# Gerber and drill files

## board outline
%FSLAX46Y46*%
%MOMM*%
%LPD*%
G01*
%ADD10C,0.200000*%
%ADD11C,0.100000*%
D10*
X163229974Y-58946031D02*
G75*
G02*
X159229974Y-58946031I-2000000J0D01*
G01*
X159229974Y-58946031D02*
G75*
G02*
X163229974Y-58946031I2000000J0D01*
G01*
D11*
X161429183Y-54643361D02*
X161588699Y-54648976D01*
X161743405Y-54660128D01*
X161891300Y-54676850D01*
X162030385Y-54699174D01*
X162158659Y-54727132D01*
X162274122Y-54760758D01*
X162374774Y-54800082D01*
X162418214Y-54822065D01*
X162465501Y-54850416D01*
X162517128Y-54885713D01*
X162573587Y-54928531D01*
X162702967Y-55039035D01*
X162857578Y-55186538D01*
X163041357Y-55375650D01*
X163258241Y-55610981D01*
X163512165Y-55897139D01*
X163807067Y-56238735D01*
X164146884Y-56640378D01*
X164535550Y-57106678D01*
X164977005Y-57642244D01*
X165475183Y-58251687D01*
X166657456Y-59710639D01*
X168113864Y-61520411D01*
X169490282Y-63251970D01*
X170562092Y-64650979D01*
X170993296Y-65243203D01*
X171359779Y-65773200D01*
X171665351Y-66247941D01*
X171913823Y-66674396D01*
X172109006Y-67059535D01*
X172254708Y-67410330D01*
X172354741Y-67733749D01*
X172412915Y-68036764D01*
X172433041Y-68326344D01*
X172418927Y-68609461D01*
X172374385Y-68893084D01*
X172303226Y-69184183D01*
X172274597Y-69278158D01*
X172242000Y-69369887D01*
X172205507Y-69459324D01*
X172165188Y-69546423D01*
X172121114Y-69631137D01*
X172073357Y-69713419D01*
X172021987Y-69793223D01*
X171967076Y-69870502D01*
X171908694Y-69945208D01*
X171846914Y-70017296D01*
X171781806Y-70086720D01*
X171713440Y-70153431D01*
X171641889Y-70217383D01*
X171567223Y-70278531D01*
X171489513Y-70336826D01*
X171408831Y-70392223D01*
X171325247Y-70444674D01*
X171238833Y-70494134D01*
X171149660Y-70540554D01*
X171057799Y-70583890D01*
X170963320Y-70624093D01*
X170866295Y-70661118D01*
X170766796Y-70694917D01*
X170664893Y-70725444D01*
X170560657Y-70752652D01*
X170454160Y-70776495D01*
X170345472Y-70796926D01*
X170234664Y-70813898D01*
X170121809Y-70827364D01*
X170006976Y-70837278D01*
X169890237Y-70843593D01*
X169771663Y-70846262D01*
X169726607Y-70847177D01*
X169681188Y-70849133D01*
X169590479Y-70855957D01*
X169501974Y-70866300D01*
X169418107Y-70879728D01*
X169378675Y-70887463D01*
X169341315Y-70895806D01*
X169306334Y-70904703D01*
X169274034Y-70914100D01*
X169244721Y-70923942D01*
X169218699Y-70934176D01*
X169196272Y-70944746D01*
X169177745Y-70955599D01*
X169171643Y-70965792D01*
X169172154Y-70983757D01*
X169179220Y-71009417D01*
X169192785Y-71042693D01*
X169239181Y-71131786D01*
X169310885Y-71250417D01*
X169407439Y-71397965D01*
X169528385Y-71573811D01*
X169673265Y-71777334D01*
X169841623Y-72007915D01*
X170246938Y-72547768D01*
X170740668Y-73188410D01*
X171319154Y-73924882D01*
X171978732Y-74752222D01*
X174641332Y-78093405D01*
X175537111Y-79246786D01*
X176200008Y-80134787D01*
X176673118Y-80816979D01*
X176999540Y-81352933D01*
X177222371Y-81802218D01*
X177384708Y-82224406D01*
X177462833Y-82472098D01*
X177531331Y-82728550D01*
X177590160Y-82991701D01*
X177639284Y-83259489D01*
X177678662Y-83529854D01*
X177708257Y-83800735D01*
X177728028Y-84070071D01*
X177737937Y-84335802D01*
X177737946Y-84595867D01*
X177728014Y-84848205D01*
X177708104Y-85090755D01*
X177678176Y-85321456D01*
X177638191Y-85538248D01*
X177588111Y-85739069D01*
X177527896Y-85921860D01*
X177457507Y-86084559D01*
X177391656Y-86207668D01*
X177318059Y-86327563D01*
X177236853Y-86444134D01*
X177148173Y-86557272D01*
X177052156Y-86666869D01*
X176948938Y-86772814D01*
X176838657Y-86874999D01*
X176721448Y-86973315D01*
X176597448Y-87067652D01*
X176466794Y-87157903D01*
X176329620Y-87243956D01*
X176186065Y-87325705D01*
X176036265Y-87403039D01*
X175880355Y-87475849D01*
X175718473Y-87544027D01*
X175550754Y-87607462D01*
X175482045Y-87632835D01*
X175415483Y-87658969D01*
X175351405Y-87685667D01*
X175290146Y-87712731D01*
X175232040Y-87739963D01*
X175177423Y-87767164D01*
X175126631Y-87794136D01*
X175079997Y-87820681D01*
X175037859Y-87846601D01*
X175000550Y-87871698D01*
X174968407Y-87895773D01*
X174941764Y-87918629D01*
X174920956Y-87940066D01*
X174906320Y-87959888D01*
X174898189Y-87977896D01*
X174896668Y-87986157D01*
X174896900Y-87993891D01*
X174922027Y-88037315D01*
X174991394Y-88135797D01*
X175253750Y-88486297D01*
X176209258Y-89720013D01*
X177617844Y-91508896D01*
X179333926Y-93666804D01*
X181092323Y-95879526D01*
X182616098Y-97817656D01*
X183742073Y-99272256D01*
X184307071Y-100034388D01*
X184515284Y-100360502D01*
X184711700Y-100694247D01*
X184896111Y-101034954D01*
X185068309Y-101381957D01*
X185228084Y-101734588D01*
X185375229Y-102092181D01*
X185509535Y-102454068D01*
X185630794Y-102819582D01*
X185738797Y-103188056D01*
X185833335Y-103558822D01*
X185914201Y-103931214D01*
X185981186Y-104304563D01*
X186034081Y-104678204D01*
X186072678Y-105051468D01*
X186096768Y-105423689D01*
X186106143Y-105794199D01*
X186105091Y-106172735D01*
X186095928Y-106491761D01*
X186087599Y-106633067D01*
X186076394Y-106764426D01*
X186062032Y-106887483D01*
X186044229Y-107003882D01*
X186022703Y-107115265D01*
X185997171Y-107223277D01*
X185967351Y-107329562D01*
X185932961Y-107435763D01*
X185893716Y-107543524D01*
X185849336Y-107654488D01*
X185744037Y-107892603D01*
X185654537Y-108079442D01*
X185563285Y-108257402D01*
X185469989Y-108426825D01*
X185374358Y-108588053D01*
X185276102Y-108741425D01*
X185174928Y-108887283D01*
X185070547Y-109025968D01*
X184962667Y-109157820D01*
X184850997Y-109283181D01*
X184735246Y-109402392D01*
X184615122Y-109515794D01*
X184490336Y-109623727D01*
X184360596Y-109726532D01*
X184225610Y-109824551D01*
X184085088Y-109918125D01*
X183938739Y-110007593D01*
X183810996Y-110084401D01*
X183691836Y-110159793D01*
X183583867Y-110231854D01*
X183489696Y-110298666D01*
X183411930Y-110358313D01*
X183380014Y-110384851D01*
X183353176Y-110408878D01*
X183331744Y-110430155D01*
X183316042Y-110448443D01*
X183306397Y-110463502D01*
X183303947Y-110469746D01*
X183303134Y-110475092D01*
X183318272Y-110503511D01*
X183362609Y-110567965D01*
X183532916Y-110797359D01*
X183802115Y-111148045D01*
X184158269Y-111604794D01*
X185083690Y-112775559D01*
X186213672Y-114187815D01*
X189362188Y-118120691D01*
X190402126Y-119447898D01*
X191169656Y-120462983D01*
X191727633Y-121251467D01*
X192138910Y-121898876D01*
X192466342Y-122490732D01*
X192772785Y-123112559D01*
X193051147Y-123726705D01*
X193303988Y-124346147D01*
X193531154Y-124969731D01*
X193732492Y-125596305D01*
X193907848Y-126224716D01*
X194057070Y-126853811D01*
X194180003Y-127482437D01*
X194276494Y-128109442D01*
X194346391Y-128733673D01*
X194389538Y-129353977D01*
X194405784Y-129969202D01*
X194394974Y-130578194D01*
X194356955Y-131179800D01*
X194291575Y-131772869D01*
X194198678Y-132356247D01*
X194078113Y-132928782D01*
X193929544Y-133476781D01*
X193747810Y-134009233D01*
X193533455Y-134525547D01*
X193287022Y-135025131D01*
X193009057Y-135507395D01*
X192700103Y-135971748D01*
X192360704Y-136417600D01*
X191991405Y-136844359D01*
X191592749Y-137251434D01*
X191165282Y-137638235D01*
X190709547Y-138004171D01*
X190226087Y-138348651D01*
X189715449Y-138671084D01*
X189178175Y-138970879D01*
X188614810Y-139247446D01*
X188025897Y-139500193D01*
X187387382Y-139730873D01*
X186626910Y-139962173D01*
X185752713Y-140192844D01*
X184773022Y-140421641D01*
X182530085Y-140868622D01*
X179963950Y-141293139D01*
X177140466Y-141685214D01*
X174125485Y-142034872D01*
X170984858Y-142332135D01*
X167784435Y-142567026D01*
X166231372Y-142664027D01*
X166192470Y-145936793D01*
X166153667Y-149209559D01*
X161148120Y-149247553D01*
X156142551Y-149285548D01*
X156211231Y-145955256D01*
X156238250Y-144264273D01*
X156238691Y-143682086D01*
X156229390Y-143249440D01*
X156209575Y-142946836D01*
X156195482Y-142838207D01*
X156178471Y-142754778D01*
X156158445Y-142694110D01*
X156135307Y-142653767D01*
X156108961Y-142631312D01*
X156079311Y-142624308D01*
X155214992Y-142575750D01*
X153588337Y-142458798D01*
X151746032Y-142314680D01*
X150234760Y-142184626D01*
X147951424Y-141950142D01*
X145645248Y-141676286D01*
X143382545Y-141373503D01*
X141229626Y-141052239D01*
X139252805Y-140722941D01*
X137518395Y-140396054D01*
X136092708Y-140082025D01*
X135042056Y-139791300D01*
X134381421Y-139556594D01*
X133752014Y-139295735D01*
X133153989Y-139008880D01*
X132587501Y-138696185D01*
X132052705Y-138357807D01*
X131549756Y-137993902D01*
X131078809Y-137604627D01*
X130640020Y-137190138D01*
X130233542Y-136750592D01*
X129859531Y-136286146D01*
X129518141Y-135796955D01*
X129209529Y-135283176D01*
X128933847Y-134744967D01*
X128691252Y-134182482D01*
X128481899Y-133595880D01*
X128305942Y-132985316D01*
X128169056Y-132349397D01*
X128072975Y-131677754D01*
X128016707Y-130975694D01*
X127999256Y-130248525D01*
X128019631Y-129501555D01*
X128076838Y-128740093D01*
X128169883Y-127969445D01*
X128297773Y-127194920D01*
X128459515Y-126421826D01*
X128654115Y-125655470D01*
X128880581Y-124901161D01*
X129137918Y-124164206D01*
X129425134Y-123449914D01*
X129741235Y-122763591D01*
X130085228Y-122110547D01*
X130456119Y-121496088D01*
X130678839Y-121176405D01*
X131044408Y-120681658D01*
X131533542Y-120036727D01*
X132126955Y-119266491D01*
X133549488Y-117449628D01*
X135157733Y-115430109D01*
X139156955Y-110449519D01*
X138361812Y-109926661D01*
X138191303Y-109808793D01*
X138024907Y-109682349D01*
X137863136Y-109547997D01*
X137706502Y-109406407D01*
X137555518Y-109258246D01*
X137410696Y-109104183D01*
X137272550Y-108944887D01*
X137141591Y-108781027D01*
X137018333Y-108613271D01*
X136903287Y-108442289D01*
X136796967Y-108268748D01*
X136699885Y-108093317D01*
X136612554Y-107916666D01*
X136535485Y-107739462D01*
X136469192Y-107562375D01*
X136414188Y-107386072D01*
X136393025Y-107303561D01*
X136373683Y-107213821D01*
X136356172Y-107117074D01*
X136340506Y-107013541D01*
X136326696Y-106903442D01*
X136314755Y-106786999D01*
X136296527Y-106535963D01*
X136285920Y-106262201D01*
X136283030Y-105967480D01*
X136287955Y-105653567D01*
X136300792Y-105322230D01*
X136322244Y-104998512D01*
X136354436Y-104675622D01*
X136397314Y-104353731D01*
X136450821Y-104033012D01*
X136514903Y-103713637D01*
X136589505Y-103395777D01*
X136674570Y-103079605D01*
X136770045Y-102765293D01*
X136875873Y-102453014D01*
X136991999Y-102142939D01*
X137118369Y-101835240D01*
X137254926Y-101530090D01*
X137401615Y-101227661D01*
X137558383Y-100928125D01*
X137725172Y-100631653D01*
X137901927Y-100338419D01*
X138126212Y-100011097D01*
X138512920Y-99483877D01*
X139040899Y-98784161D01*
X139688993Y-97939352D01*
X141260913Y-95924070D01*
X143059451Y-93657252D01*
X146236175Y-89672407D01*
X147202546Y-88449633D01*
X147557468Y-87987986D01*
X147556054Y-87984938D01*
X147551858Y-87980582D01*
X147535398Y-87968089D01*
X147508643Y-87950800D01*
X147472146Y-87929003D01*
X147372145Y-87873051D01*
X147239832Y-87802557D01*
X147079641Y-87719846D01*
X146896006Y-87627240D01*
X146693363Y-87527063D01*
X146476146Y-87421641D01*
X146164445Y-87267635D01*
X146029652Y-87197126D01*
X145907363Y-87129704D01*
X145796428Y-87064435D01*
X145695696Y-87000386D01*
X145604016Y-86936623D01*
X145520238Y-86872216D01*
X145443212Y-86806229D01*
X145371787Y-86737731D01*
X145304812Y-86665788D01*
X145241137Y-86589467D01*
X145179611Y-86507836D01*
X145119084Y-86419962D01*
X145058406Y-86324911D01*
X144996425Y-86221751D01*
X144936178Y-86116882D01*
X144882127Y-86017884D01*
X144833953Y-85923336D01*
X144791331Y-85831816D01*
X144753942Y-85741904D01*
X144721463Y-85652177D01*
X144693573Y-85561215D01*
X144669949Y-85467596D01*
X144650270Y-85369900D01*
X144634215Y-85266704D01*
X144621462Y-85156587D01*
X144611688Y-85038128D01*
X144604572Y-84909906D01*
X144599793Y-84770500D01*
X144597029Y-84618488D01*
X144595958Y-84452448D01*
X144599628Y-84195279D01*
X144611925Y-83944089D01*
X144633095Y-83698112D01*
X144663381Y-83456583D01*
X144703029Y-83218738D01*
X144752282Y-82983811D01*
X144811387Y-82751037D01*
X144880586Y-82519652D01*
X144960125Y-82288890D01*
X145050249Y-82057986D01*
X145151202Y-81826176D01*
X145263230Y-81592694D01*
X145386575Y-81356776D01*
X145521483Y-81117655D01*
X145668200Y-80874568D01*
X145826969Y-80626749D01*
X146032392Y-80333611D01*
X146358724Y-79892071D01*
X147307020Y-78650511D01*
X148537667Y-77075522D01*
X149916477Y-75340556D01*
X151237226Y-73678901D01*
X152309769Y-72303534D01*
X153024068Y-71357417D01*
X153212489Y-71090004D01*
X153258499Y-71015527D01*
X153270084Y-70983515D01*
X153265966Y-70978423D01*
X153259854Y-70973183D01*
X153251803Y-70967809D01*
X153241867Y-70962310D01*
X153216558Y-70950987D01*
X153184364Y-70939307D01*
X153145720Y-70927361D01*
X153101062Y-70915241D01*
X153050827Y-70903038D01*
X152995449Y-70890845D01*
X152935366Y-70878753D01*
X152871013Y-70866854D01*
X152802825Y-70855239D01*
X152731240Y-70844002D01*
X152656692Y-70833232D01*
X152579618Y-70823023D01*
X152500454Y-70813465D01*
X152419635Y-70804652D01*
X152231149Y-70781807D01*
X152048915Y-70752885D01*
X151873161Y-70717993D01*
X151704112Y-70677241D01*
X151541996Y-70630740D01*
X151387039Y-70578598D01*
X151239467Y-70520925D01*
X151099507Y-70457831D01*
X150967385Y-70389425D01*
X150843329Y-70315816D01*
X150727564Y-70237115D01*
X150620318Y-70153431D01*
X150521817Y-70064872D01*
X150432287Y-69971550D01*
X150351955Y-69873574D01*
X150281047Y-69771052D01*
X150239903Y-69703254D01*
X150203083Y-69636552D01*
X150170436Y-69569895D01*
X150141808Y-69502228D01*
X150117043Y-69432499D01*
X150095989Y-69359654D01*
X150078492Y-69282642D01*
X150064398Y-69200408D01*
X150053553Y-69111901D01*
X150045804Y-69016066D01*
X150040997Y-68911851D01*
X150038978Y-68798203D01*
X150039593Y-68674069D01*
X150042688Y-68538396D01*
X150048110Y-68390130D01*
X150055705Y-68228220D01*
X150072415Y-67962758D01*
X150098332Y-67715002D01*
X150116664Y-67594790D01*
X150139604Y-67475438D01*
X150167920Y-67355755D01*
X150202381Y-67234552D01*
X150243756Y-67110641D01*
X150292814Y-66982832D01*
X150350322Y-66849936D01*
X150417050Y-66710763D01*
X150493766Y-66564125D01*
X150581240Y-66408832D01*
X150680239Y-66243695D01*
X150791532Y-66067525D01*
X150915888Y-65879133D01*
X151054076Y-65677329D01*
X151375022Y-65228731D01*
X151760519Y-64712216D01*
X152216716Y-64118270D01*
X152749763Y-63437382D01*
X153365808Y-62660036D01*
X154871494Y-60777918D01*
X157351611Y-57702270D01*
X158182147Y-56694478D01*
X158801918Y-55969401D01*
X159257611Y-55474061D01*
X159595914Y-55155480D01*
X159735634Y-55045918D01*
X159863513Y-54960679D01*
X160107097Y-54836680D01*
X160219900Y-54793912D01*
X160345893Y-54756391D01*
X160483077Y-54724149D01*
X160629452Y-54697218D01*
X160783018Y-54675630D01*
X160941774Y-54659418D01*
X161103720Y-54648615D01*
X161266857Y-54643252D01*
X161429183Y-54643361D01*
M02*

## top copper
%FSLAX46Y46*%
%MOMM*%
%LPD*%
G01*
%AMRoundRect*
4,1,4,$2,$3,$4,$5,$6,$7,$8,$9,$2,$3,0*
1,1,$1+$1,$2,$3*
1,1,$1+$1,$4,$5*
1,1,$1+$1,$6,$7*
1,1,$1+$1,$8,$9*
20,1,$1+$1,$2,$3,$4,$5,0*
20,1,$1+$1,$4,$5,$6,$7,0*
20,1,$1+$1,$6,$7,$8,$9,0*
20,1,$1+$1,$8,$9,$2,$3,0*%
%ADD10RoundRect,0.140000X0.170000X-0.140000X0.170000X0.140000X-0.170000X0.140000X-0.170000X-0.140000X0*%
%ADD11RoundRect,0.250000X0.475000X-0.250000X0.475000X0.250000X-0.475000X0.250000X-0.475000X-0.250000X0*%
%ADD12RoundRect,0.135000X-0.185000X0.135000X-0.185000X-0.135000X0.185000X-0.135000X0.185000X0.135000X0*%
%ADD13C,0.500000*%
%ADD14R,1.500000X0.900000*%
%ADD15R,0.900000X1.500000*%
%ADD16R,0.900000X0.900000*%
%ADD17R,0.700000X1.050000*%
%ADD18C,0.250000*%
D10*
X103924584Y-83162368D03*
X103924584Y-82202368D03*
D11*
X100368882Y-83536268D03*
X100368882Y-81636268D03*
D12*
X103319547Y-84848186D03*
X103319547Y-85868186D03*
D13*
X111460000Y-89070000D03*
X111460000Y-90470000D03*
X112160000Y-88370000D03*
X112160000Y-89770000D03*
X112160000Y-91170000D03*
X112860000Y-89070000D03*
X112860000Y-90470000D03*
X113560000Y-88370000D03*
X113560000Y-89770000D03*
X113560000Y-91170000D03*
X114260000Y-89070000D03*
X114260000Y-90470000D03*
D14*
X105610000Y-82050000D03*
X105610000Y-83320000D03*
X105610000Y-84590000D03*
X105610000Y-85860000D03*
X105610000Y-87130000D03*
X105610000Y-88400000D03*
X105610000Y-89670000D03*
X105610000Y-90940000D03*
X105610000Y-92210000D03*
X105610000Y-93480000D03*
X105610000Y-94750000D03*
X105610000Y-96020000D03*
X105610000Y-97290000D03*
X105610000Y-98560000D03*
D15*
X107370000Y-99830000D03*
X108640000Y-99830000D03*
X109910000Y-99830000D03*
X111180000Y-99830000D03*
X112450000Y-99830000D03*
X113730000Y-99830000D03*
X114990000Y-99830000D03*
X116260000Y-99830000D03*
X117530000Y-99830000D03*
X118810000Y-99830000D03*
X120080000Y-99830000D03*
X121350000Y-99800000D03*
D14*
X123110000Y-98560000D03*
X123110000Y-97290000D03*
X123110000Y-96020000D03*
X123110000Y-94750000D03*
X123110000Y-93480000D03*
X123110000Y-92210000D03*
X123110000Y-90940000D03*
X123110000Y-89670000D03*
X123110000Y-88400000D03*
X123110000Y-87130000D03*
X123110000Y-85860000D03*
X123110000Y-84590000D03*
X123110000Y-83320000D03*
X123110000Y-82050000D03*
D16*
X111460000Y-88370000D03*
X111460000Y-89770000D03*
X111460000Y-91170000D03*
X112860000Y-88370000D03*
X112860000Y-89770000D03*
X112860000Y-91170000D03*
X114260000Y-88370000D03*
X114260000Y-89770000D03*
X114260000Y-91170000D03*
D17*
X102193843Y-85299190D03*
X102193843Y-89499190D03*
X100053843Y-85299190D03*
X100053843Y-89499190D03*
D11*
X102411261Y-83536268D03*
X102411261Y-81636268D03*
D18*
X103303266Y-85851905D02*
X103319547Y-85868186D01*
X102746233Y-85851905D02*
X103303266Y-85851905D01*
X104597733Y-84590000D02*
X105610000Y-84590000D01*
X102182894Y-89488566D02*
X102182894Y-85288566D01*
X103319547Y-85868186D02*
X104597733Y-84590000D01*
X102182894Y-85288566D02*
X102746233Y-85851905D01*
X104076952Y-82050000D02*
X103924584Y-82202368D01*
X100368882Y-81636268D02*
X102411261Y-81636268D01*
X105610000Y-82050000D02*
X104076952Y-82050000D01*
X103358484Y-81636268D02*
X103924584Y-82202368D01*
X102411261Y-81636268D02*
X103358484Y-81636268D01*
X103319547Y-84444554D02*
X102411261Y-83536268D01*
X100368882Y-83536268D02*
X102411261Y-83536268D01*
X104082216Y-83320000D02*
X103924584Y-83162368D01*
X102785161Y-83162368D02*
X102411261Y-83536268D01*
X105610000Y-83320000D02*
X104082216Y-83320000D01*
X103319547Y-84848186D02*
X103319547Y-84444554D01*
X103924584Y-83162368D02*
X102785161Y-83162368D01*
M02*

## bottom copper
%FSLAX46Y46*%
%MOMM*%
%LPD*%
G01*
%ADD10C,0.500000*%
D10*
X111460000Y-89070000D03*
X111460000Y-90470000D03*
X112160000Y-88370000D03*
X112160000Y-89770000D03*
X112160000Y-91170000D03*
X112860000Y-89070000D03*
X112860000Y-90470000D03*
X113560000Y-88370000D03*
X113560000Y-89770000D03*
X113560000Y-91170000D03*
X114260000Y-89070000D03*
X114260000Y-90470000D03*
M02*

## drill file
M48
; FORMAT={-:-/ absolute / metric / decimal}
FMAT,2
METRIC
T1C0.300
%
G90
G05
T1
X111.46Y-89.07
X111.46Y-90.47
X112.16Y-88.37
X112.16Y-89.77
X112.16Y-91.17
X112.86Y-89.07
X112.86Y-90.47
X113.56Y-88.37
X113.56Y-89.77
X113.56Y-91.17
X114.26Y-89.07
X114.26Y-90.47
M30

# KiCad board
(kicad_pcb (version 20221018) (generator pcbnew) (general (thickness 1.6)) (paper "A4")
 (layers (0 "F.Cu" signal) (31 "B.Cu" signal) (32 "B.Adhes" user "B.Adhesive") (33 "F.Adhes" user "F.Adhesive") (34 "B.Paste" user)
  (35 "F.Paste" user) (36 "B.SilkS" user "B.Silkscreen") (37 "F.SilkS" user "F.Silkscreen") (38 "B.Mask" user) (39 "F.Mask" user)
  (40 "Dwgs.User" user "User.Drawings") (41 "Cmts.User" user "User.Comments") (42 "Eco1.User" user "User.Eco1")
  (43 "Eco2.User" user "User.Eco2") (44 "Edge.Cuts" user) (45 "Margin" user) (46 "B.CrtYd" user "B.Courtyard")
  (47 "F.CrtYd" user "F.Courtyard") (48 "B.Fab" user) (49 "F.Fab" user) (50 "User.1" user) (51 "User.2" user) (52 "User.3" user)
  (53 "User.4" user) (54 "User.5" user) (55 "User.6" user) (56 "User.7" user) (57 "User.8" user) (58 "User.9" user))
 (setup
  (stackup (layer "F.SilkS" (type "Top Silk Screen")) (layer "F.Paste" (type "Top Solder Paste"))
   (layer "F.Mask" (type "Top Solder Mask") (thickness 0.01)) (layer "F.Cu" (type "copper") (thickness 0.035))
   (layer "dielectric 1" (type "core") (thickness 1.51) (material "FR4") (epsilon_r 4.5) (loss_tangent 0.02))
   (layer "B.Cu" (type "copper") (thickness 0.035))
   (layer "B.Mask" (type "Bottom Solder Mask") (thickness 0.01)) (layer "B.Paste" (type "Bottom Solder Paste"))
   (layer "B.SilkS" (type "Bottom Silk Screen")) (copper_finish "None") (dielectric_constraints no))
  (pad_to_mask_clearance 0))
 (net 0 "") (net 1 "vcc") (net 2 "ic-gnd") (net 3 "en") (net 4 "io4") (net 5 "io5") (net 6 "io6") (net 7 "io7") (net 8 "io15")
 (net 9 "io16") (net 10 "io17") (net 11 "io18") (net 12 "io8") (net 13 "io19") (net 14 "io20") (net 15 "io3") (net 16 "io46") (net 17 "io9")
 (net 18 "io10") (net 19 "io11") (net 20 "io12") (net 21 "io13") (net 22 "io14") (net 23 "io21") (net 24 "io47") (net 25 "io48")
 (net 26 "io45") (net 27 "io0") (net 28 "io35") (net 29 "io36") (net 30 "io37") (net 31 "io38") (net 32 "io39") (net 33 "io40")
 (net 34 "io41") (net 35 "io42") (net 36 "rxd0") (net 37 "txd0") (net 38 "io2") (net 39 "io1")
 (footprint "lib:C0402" (layer "F.Cu") (at 103.924584 82.682368 90)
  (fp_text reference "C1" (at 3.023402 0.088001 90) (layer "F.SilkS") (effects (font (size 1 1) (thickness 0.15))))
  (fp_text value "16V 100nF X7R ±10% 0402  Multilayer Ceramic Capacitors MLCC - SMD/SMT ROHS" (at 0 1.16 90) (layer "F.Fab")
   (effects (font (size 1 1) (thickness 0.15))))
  (pad "1" smd roundrect (at -0.48 0 90) (size 0.56 0.62) (layers "F.Cu" "F.Paste" "F.Mask") (roundrect_rratio 0.25) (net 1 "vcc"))
  (pad "2" smd roundrect (at 0.48 0 90) (size 0.56 0.62) (layers "F.Cu" "F.Paste" "F.Mask") (roundrect_rratio 0.25) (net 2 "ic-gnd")))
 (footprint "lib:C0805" (layer "F.Cu") (at 100.368882 82.586268 90)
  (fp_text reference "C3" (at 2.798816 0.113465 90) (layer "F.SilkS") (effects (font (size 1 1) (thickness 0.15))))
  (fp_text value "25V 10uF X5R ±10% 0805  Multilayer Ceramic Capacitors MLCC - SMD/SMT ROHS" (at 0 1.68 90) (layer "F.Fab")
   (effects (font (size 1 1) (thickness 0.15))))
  (pad "1" smd roundrect (at -0.95 0 90) (size 1 1.45) (layers "F.Cu" "F.Paste" "F.Mask") (roundrect_rratio 0.25) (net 1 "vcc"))
  (pad "2" smd roundrect (at 0.95 0 90) (size 1 1.45) (layers "F.Cu" "F.Paste" "F.Mask") (roundrect_rratio 0.25) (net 2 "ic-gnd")))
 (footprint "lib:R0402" (layer "F.Cu") (at 103.319547 85.358186 -90)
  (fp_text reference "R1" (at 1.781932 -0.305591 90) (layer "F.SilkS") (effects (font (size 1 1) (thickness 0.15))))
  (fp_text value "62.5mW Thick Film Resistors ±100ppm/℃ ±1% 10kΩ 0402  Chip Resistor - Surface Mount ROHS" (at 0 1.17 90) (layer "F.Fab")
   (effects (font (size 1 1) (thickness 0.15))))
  (pad "1" smd roundrect (at -0.51 0 270) (size 0.54 0.64) (layers "F.Cu" "F.Paste" "F.Mask") (roundrect_rratio 0.25) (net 1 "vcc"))
  (pad "2" smd roundrect (at 0.51 0 270) (size 0.54 0.64) (layers "F.Cu" "F.Paste" "F.Mask") (roundrect_rratio 0.25) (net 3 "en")))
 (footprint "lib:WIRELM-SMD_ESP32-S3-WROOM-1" (layer "F.Cu") (at 114.36 90.94)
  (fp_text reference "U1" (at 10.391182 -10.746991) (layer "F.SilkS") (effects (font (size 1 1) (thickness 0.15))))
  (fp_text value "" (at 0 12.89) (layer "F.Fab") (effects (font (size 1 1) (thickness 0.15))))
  (pad "" thru_hole circle (at -2.9 -1.87) (size 0.5 0.5) (drill 0.3) (layers "*.Cu" "*.Paste" "*.Mask"))
  (pad "" thru_hole circle (at -2.9 -0.47) (size 0.5 0.5) (drill 0.3) (layers "*.Cu" "*.Paste" "*.Mask"))
  (pad "" thru_hole circle (at -2.2 -2.57) (size 0.5 0.5) (drill 0.3) (layers "*.Cu" "*.Paste" "*.Mask"))
  (pad "" thru_hole circle (at -2.2 -1.17) (size 0.5 0.5) (drill 0.3) (layers "*.Cu" "*.Paste" "*.Mask"))
  (pad "" thru_hole circle (at -2.2 0.23) (size 0.5 0.5) (drill 0.3) (layers "*.Cu" "*.Paste" "*.Mask"))
  (pad "" thru_hole circle (at -1.5 -1.87) (size 0.5 0.5) (drill 0.3) (layers "*.Cu" "*.Paste" "*.Mask"))
  (pad "" thru_hole circle (at -1.5 -0.47) (size 0.5 0.5) (drill 0.3) (layers "*.Cu" "*.Paste" "*.Mask"))
  (pad "" thru_hole circle (at -0.8 -2.57) (size 0.5 0.5) (drill 0.3) (layers "*.Cu" "*.Paste" "*.Mask"))
  (pad "" thru_hole circle (at -0.8 -1.17) (size 0.5 0.5) (drill 0.3) (layers "*.Cu" "*.Paste" "*.Mask"))
  (pad "" thru_hole circle (at -0.8 0.23) (size 0.5 0.5) (drill 0.3) (layers "*.Cu" "*.Paste" "*.Mask"))
  (pad "" thru_hole circle (at -0.1 -1.87) (size 0.5 0.5) (drill 0.3) (layers "*.Cu" "*.Paste" "*.Mask"))
  (pad "" thru_hole circle (at -0.1 -0.47) (size 0.5 0.5) (drill 0.3) (layers "*.Cu" "*.Paste" "*.Mask"))
  (pad "1" smd rect (at -8.75 -8.89) (size 1.5 0.9) (layers "F.Cu" "F.Paste" "F.Mask") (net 2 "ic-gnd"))
  (pad "2" smd rect (at -8.75 -7.62) (size 1.5 0.9) (layers "F.Cu" "F.Paste" "F.Mask") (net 1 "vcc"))
  (pad "3" smd rect (at -8.75 -6.35) (size 1.5 0.9) (layers "F.Cu" "F.Paste" "F.Mask") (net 3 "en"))
  (pad "4" smd rect (at -8.75 -5.08) (size 1.5 0.9) (layers "F.Cu" "F.Paste" "F.Mask") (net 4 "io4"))
  (pad "5" smd rect (at -8.75 -3.81) (size 1.5 0.9) (layers "F.Cu" "F.Paste" "F.Mask") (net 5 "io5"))
  (pad "6" smd rect (at -8.75 -2.54) (size 1.5 0.9) (layers "F.Cu" "F.Paste" "F.Mask") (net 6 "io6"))
  (pad "7" smd rect (at -8.75 -1.27) (size 1.5 0.9) (layers "F.Cu" "F.Paste" "F.Mask") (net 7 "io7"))
  (pad "8" smd rect (at -8.75 0) (size 1.5 0.9) (layers "F.Cu" "F.Paste" "F.Mask") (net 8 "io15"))
  (pad "9" smd rect (at -8.75 1.27) (size 1.5 0.9) (layers "F.Cu" "F.Paste" "F.Mask") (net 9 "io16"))
  (pad "10" smd rect (at -8.75 2.54) (size 1.5 0.9) (layers "F.Cu" "F.Paste" "F.Mask") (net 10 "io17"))
  (pad "11" smd rect (at -8.75 3.81) (size 1.5 0.9) (layers "F.Cu" "F.Paste" "F.Mask") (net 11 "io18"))
  (pad "12" smd rect (at -8.75 5.08) (size 1.5 0.9) (layers "F.Cu" "F.Paste" "F.Mask") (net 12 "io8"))
  (pad "13" smd rect (at -8.75 6.35) (size 1.5 0.9) (layers "F.Cu" "F.Paste" "F.Mask") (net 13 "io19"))
  (pad "14" smd rect (at -8.75 7.62) (size 1.5 0.9) (layers "F.Cu" "F.Paste" "F.Mask") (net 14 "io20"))
  (pad "15" smd rect (at -6.99 8.89 90) (size 1.5 0.9) (layers "F.Cu" "F.Paste" "F.Mask") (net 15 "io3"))
  (pad "16" smd rect (at -5.72 8.89 90) (size 1.5 0.9) (layers "F.Cu" "F.Paste" "F.Mask") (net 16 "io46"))
  (pad "17" smd rect (at -4.45 8.89 90) (size 1.5 0.9) (layers "F.Cu" "F.Paste" "F.Mask") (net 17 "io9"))
  (pad "18" smd rect (at -3.18 8.89 90) (size 1.5 0.9) (layers "F.Cu" "F.Paste" "F.Mask") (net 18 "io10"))
  (pad "19" smd rect (at -1.91 8.89 90) (size 1.5 0.9) (layers "F.Cu" "F.Paste" "F.Mask") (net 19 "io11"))
  (pad "20" smd rect (at -0.63 8.89 90) (size 1.5 0.9) (layers "F.Cu" "F.Paste" "F.Mask") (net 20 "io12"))
  (pad "21" smd rect (at 0.63 8.89 90) (size 1.5 0.9) (layers "F.Cu" "F.Paste" "F.Mask") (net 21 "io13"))
  (pad "22" smd rect (at 1.9 8.89 90) (size 1.5 0.9) (layers "F.Cu" "F.Paste" "F.Mask") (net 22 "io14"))
  (pad "23" smd rect (at 3.17 8.89 90) (size 1.5 0.9) (layers "F.Cu" "F.Paste" "F.Mask") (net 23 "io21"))
  (pad "24" smd rect (at 4.45 8.89 90) (size 1.5 0.9) (layers "F.Cu" "F.Paste" "F.Mask") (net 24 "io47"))
  (pad "25" smd rect (at 5.72 8.89 90) (size 1.5 0.9) (layers "F.Cu" "F.Paste" "F.Mask") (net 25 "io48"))
  (pad "26" smd rect (at 6.99 8.86 90) (size 1.5 0.9) (layers "F.Cu" "F.Paste" "F.Mask") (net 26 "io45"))
  (pad "27" smd rect (at 8.75 7.62 180) (size 1.5 0.9) (layers "F.Cu" "F.Paste" "F.Mask") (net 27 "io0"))
  (pad "28" smd rect (at 8.75 6.35 180) (size 1.5 0.9) (layers "F.Cu" "F.Paste" "F.Mask") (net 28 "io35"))
  (pad "29" smd rect (at 8.75 5.08 180) (size 1.5 0.9) (layers "F.Cu" "F.Paste" "F.Mask") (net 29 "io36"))
  (pad "30" smd rect (at 8.75 3.81 180) (size 1.5 0.9) (layers "F.Cu" "F.Paste" "F.Mask") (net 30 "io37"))
  (pad "31" smd rect (at 8.75 2.54 180) (size 1.5 0.9) (layers "F.Cu" "F.Paste" "F.Mask") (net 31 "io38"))
  (pad "32" smd rect (at 8.75 1.27 180) (size 1.5 0.9) (layers "F.Cu" "F.Paste" "F.Mask") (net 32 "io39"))
  (pad "33" smd rect (at 8.75 0 180) (size 1.5 0.9) (layers "F.Cu" "F.Paste" "F.Mask") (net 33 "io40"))
  (pad "34" smd rect (at 8.75 -1.27 180) (size 1.5 0.9) (layers "F.Cu" "F.Paste" "F.Mask") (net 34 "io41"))
  (pad "35" smd rect (at 8.75 -2.54 180) (size 1.5 0.9) (layers "F.Cu" "F.Paste" "F.Mask") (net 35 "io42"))
  (pad "36" smd rect (at 8.75 -3.81 180) (size 1.5 0.9) (layers "F.Cu" "F.Paste" "F.Mask") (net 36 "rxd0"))
  (pad "37" smd rect (at 8.75 -5.08 180) (size 1.5 0.9) (layers "F.Cu" "F.Paste" "F.Mask") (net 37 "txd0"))
  (pad "38" smd rect (at 8.75 -6.35 180) (size 1.5 0.9) (layers "F.Cu" "F.Paste" "F.Mask") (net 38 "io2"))
  (pad "39" smd rect (at 8.75 -7.62 180) (size 1.5 0.9) (layers "F.Cu" "F.Paste" "F.Mask") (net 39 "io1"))
  (pad "40" smd rect (at 8.75 -8.89 180) (size 1.5 0.9) (layers "F.Cu" "F.Paste" "F.Mask") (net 2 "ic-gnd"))
  (pad "41" smd rect (at -2.9 -2.57 90) (size 0.9 0.9) (layers "F.Cu" "F.Paste" "F.Mask") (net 2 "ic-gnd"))
  (pad "41" smd rect (at -2.9 -1.17 90) (size 0.9 0.9) (layers "F.Cu" "F.Paste" "F.Mask") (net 2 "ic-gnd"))
  (pad "41" smd rect (at -2.9 0.23 90) (size 0.9 0.9) (layers "F.Cu" "F.Paste" "F.Mask") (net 2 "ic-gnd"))
  (pad "41" smd rect (at -1.5 -2.57 90) (size 0.9 0.9) (layers "F.Cu" "F.Paste" "F.Mask") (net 2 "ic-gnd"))
  (pad "41" smd rect (at -1.5 -1.17 90) (size 0.9 0.9) (layers "F.Cu" "F.Paste" "F.Mask") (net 2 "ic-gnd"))
  (pad "41" smd rect (at -1.5 0.23 90) (size 0.9 0.9) (layers "F.Cu" "F.Paste" "F.Mask") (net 2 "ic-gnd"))
  (pad "41" smd rect (at -0.1 -2.57 90) (size 0.9 0.9) (layers "F.Cu" "F.Paste" "F.Mask") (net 2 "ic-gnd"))
  (pad "41" smd rect (at -0.1 -1.17 90) (size 0.9 0.9) (layers "F.Cu" "F.Paste" "F.Mask") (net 2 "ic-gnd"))
  (pad "41" smd rect (at -0.1 0.23 90) (size 0.9 0.9) (layers "F.Cu" "F.Paste" "F.Mask") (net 2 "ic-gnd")))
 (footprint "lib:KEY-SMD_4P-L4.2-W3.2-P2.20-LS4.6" (layer "F.Cu") (at 101.123843 87.39919 -90)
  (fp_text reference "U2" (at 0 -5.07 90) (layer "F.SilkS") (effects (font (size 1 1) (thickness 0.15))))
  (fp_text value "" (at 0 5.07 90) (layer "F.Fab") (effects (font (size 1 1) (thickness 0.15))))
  (pad "1" smd rect (at -2.1 -1.07 270) (size 1.05 0.7) (layers "F.Cu" "F.Paste" "F.Mask") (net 3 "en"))
  (pad "2" smd rect (at 2.1 -1.07 270) (size 1.05 0.7) (layers "F.Cu" "F.Paste" "F.Mask") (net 3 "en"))
  (pad "3" smd rect (at -2.1 1.07 270) (size 1.05 0.7) (layers "F.Cu" "F.Paste" "F.Mask") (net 2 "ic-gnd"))
  (pad "4" smd rect (at 2.1 1.07 270) (size 1.05 0.7) (layers "F.Cu" "F.Paste" "F.Mask") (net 2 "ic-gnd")))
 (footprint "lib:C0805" (layer "F.Cu") (at 102.411261 82.586268 90)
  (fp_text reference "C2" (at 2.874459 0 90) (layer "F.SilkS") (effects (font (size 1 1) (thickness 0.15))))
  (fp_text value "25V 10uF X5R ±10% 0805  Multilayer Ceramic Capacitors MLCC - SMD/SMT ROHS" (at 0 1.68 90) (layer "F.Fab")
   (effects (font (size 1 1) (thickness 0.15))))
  (pad "1" smd roundrect (at -0.95 0 90) (size 1 1.45) (layers "F.Cu" "F.Paste" "F.Mask") (roundrect_rratio 0.25) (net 1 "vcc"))
  (pad "2" smd roundrect (at 0.95 0 90) (size 1 1.45) (layers "F.Cu" "F.Paste" "F.Mask") (roundrect_rratio 0.25) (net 2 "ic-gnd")))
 (gr_circle (center 161.229974 58.946031) (end 163.229974 58.946031) (stroke (width 0.2) (type default)) (fill none) (layer "Edge.Cuts"))
 (gr_poly
  (pts (xy 161.429183 54.643361) (xy 161.588699 54.648976) (xy 161.743405 54.660128) (xy 161.8913 54.67685) (xy 162.030385 54.699174)
   (xy 162.158659 54.727132) (xy 162.274122 54.760758) (xy 162.374774 54.800082) (xy 162.418214 54.822065) (xy 162.465501 54.850416)
   (xy 162.517128 54.885713) (xy 162.573587 54.928531) (xy 162.702967 55.039035) (xy 162.857578 55.186538) (xy 163.041357 55.37565)
   (xy 163.258241 55.610981) (xy 163.512165 55.897139) (xy 163.807067 56.238735) (xy 164.146884 56.640378) (xy 164.53555 57.106678)
   (xy 164.977005 57.642244) (xy 165.475183 58.251687) (xy 166.657456 59.710639) (xy 168.113864 61.520411) (xy 169.490282 63.25197)
   (xy 170.562092 64.650979) (xy 170.993296 65.243203) (xy 171.359779 65.7732) (xy 171.665351 66.247941) (xy 171.913823 66.674396)
   (xy 172.109006 67.059535) (xy 172.254708 67.41033) (xy 172.354741 67.733749) (xy 172.412915 68.036764) (xy 172.433041 68.326344)
   (xy 172.418927 68.609461) (xy 172.374385 68.893084) (xy 172.303226 69.184183) (xy 172.274597 69.278158) (xy 172.242 69.369887)
   (xy 172.205507 69.459324) (xy 172.165188 69.546423) (xy 172.121114 69.631137) (xy 172.073357 69.713419) (xy 172.021987 69.793223)
   (xy 171.967076 69.870502) (xy 171.908694 69.945208) (xy 171.846914 70.017296) (xy 171.781806 70.08672) (xy 171.71344 70.153431)
   (xy 171.641889 70.217383) (xy 171.567223 70.278531) (xy 171.489513 70.336826) (xy 171.408831 70.392223) (xy 171.325247 70.444674)
   (xy 171.238833 70.494134) (xy 171.14966 70.540554) (xy 171.057799 70.58389) (xy 170.96332 70.624093) (xy 170.866295 70.661118)
   (xy 170.766796 70.694917) (xy 170.664893 70.725444) (xy 170.560657 70.752652) (xy 170.45416 70.776495) (xy 170.345472 70.796926)
   (xy 170.234664 70.813898) (xy 170.121809 70.827364) (xy 170.006976 70.837278) (xy 169.890237 70.843593) (xy 169.771663 70.846262)
   (xy 169.726607 70.847177) (xy 169.681188 70.849133) (xy 169.590479 70.855957) (xy 169.501974 70.8663) (xy 169.418107 70.879728)
   (xy 169.378675 70.887463) (xy 169.341315 70.895806) (xy 169.306334 70.904703) (xy 169.274034 70.9141) (xy 169.244721 70.923942)
   (xy 169.218699 70.934176) (xy 169.196272 70.944746) (xy 169.177745 70.955599) (xy 169.171643 70.965792) (xy 169.172154 70.983757)
   (xy 169.17922 71.009417) (xy 169.192785 71.042693) (xy 169.239181 71.131786) (xy 169.310885 71.250417) (xy 169.407439 71.397965)
   (xy 169.528385 71.573811) (xy 169.673265 71.777334) (xy 169.841623 72.007915) (xy 170.246938 72.547768) (xy 170.740668 73.18841)
   (xy 171.319154 73.924882) (xy 171.978732 74.752222) (xy 174.641332 78.093405) (xy 175.537111 79.246786) (xy 176.200008 80.134787)
   (xy 176.673118 80.816979) (xy 176.99954 81.352933) (xy 177.222371 81.802218) (xy 177.384708 82.224406) (xy 177.462833 82.472098)
   (xy 177.531331 82.72855) (xy 177.59016 82.991701) (xy 177.639284 83.259489) (xy 177.678662 83.529854) (xy 177.708257 83.800735)
   (xy 177.728028 84.070071) (xy 177.737937 84.335802) (xy 177.737946 84.595867) (xy 177.728014 84.848205) (xy 177.708104 85.090755)
   (xy 177.678176 85.321456) (xy 177.638191 85.538248) (xy 177.588111 85.739069) (xy 177.527896 85.92186) (xy 177.457507 86.084559)
   (xy 177.391656 86.207668) (xy 177.318059 86.327563) (xy 177.236853 86.444134) (xy 177.148173 86.557272) (xy 177.052156 86.666869)
   (xy 176.948938 86.772814) (xy 176.838657 86.874999) (xy 176.721448 86.973315) (xy 176.597448 87.067652) (xy 176.466794 87.157903)
   (xy 176.32962 87.243956) (xy 176.186065 87.325705) (xy 176.036265 87.403039) (xy 175.880355 87.475849) (xy 175.718473 87.544027)
   (xy 175.550754 87.607462) (xy 175.482045 87.632835) (xy 175.415483 87.658969) (xy 175.351405 87.685667) (xy 175.290146 87.712731)
   (xy 175.23204 87.739963) (xy 175.177423 87.767164) (xy 175.126631 87.794136) (xy 175.079997 87.820681) (xy 175.037859 87.846601)
   (xy 175.00055 87.871698) (xy 174.968407 87.895773) (xy 174.941764 87.918629) (xy 174.920956 87.940066) (xy 174.90632 87.959888)
   (xy 174.898189 87.977896) (xy 174.896668 87.986157) (xy 174.8969 87.993891) (xy 174.922027 88.037315) (xy 174.991394 88.135797)
   (xy 175.25375 88.486297) (xy 176.209258 89.720013) (xy 177.617844 91.508896) (xy 179.333926 93.666804) (xy 181.092323 95.879526)
   (xy 182.616098 97.817656) (xy 183.742073 99.272256) (xy 184.307071 100.034388) (xy 184.515284 100.360502) (xy 184.7117 100.694247)
   (xy 184.896111 101.034954) (xy 185.068309 101.381957) (xy 185.228084 101.734588) (xy 185.375229 102.092181) (xy 185.509535 102.454068)
   (xy 185.630794 102.819582) (xy 185.738797 103.188056) (xy 185.833335 103.558822) (xy 185.914201 103.931214) (xy 185.981186 104.304563)
   (xy 186.034081 104.678204) (xy 186.072678 105.051468) (xy 186.096768 105.423689) (xy 186.106143 105.794199) (xy 186.105091 106.172735)
   (xy 186.095928 106.491761) (xy 186.087599 106.633067) (xy 186.076394 106.764426) (xy 186.062032 106.887483) (xy 186.044229 107.003882)
   (xy 186.022703 107.115265) (xy 185.997171 107.223277) (xy 185.967351 107.329562) (xy 185.932961 107.435763) (xy 185.893716 107.543524)
   (xy 185.849336 107.654488) (xy 185.744037 107.892603) (xy 185.654537 108.079442) (xy 185.563285 108.257402) (xy 185.469989 108.426825)
   (xy 185.374358 108.588053) (xy 185.276102 108.741425) (xy 185.174928 108.887283) (xy 185.070547 109.025968) (xy 184.962667 109.15782)
   (xy 184.850997 109.283181) (xy 184.735246 109.402392) (xy 184.615122 109.515794) (xy 184.490336 109.623727) (xy 184.360596 109.726532)
   (xy 184.22561 109.824551) (xy 184.085088 109.918125) (xy 183.938739 110.007593) (xy 183.810996 110.084401) (xy 183.691836 110.159793)
   (xy 183.583867 110.231854) (xy 183.489696 110.298666) (xy 183.41193 110.358313) (xy 183.380014 110.384851) (xy 183.353176 110.408878)
   (xy 183.331744 110.430155) (xy 183.316042 110.448443) (xy 183.306397 110.463502) (xy 183.303947 110.469746) (xy 183.303134 110.475092)
   (xy 183.318272 110.503511) (xy 183.362609 110.567965) (xy 183.532916 110.797359) (xy 183.802115 111.148045) (xy 184.158269 111.604794)
   (xy 185.08369 112.775559) (xy 186.213672 114.187815) (xy 189.362188 118.120691) (xy 190.402126 119.447898) (xy 191.169656 120.462983)
   (xy 191.727633 121.251467) (xy 192.13891 121.898876) (xy 192.466342 122.490732) (xy 192.772785 123.112559) (xy 193.051147 123.726705)
   (xy 193.303988 124.346147) (xy 193.531154 124.969731) (xy 193.732492 125.596305) (xy 193.907848 126.224716) (xy 194.05707 126.853811)
   (xy 194.180003 127.482437) (xy 194.276494 128.109442) (xy 194.346391 128.733673) (xy 194.389538 129.353977) (xy 194.405784 129.969202)
   (xy 194.394974 130.578194) (xy 194.356955 131.1798) (xy 194.291575 131.772869) (xy 194.198678 132.356247) (xy 194.078113 132.928782)
   (xy 193.929544 133.476781) (xy 193.74781 134.009233) (xy 193.533455 134.525547) (xy 193.287022 135.025131) (xy 193.009057 135.507395)
   (xy 192.700103 135.971748) (xy 192.360704 136.4176) (xy 191.991405 136.844359) (xy 191.592749 137.251434) (xy 191.165282 137.638235)
   (xy 190.709547 138.004171) (xy 190.226087 138.348651) (xy 189.715449 138.671084) (xy 189.178175 138.970879) (xy 188.61481 139.247446)
   (xy 188.025897 139.500193) (xy 187.387382 139.730873) (xy 186.62691 139.962173) (xy 185.752713 140.192844) (xy 184.773022 140.421641)
   (xy 182.530085 140.868622) (xy 179.96395 141.293139) (xy 177.140466 141.685214) (xy 174.125485 142.034872) (xy 170.984858 142.332135)
   (xy 167.784435 142.567026) (xy 166.231372 142.664027) (xy 166.19247 145.936793) (xy 166.153667 149.209559) (xy 161.14812 149.247553)
   (xy 156.142551 149.285548) (xy 156.211231 145.955256) (xy 156.23825 144.264273) (xy 156.238691 143.682086) (xy 156.22939 143.24944)
   (xy 156.209575 142.946836) (xy 156.195482 142.838207) (xy 156.178471 142.754778) (xy 156.158445 142.69411) (xy 156.135307 142.653767)
   (xy 156.108961 142.631312) (xy 156.079311 142.624308) (xy 155.214992 142.57575) (xy 153.588337 142.458798) (xy 151.746032 142.31468)
   (xy 150.23476 142.184626) (xy 147.951424 141.950142) (xy 145.645248 141.676286) (xy 143.382545 141.373503) (xy 141.229626 141.052239)
   (xy 139.252805 140.722941) (xy 137.518395 140.396054) (xy 136.092708 140.082025) (xy 135.042056 139.7913) (xy 134.381421 139.556594)
   (xy 133.752014 139.295735) (xy 133.153989 139.00888) (xy 132.587501 138.696185) (xy 132.052705 138.357807) (xy 131.549756 137.993902)
   (xy 131.078809 137.604627) (xy 130.64002 137.190138) (xy 130.233542 136.750592) (xy 129.859531 136.286146) (xy 129.518141 135.796955)
   (xy 129.209529 135.283176) (xy 128.933847 134.744967) (xy 128.691252 134.182482) (xy 128.481899 133.59588) (xy 128.305942 132.985316)
   (xy 128.169056 132.349397) (xy 128.072975 131.677754) (xy 128.016707 130.975694) (xy 127.999256 130.248525) (xy 128.019631 129.501555)
   (xy 128.076838 128.740093) (xy 128.169883 127.969445) (xy 128.297773 127.19492) (xy 128.459515 126.421826) (xy 128.654115 125.65547)
   (xy 128.880581 124.901161) (xy 129.137918 124.164206) (xy 129.425134 123.449914) (xy 129.741235 122.763591) (xy 130.085228 122.110547)
   (xy 130.456119 121.496088) (xy 130.678839 121.176405) (xy 131.044408 120.681658) (xy 131.533542 120.036727) (xy 132.126955 119.266491)
   (xy 133.549488 117.449628) (xy 135.157733 115.430109) (xy 139.156955 110.449519) (xy 138.361812 109.926661) (xy 138.191303 109.808793)
   (xy 138.024907 109.682349) (xy 137.863136 109.547997) (xy 137.706502 109.406407) (xy 137.555518 109.258246) (xy 137.410696 109.104183)
   (xy 137.27255 108.944887) (xy 137.141591 108.781027) (xy 137.018333 108.613271) (xy 136.903287 108.442289) (xy 136.796967 108.268748)
   (xy 136.699885 108.093317) (xy 136.612554 107.916666) (xy 136.535485 107.739462) (xy 136.469192 107.562375) (xy 136.414188 107.386072)
   (xy 136.393025 107.303561) (xy 136.373683 107.213821) (xy 136.356172 107.117074) (xy 136.340506 107.013541) (xy 136.326696 106.903442)
   (xy 136.314755 106.786999) (xy 136.296527 106.535963) (xy 136.28592 106.262201) (xy 136.28303 105.96748) (xy 136.287955 105.653567)
   (xy 136.300792 105.32223) (xy 136.322244 104.998512) (xy 136.354436 104.675622) (xy 136.397314 104.353731) (xy 136.450821 104.033012)
   (xy 136.514903 103.713637) (xy 136.589505 103.395777) (xy 136.67457 103.079605) (xy 136.770045 102.765293) (xy 136.875873 102.453014)
   (xy 136.991999 102.142939) (xy 137.118369 101.83524) (xy 137.254926 101.53009) (xy 137.401615 101.227661) (xy 137.558383 100.928125)
   (xy 137.725172 100.631653) (xy 137.901927 100.338419) (xy 138.126212 100.011097) (xy 138.51292 99.483877) (xy 139.040899 98.784161)
   (xy 139.688993 97.939352) (xy 141.260913 95.92407) (xy 143.059451 93.657252) (xy 146.236175 89.672407) (xy 147.202546 88.449633)
   (xy 147.557468 87.987986) (xy 147.556054 87.984938) (xy 147.551858 87.980582) (xy 147.535398 87.968089) (xy 147.508643 87.9508)
   (xy 147.472146 87.929003) (xy 147.372145 87.873051) (xy 147.239832 87.802557) (xy 147.079641 87.719846) (xy 146.896006 87.62724)
   (xy 146.693363 87.527063) (xy 146.476146 87.421641) (xy 146.164445 87.267635) (xy 146.029652 87.197126) (xy 145.907363 87.129704)
   (xy 145.796428 87.064435) (xy 145.695696 87.000386) (xy 145.604016 86.936623) (xy 145.520238 86.872216) (xy 145.443212 86.806229)
   (xy 145.371787 86.737731) (xy 145.304812 86.665788) (xy 145.241137 86.589467) (xy 145.179611 86.507836) (xy 145.119084 86.419962)
   (xy 145.058406 86.324911) (xy 144.996425 86.221751) (xy 144.936178 86.116882) (xy 144.882127 86.017884) (xy 144.833953 85.923336)
   (xy 144.791331 85.831816) (xy 144.753942 85.741904) (xy 144.721463 85.652177) (xy 144.693573 85.561215) (xy 144.669949 85.467596)
   (xy 144.65027 85.3699) (xy 144.634215 85.266704) (xy 144.621462 85.156587) (xy 144.611688 85.038128) (xy 144.604572 84.909906)
   (xy 144.599793 84.7705) (xy 144.597029 84.618488) (xy 144.595958 84.452448) (xy 144.599628 84.195279) (xy 144.611925 83.944089)
   (xy 144.633095 83.698112) (xy 144.663381 83.456583) (xy 144.703029 83.218738) (xy 144.752282 82.983811) (xy 144.811387 82.751037)
   (xy 144.880586 82.519652) (xy 144.960125 82.28889) (xy 145.050249 82.057986) (xy 145.151202 81.826176) (xy 145.26323 81.592694)
   (xy 145.386575 81.356776) (xy 145.521483 81.117655) (xy 145.6682 80.874568) (xy 145.826969 80.626749) (xy 146.032392 80.333611)
   (xy 146.358724 79.892071) (xy 147.30702 78.650511) (xy 148.537667 77.075522) (xy 149.916477 75.340556) (xy 151.237226 73.678901)
   (xy 152.309769 72.303534) (xy 153.024068 71.357417) (xy 153.212489 71.090004) (xy 153.258499 71.015527) (xy 153.270084 70.983515)
   (xy 153.265966 70.978423) (xy 153.259854 70.973183) (xy 153.251803 70.967809) (xy 153.241867 70.96231) (xy 153.216558 70.950987)
   (xy 153.184364 70.939307) (xy 153.14572 70.927361) (xy 153.101062 70.915241) (xy 153.050827 70.903038) (xy 152.995449 70.890845)
   (xy 152.935366 70.878753) (xy 152.871013 70.866854) (xy 152.802825 70.855239) (xy 152.73124 70.844002) (xy 152.656692 70.833232)
   (xy 152.579618 70.823023) (xy 152.500454 70.813465) (xy 152.419635 70.804652) (xy 152.231149 70.781807) (xy 152.048915 70.752885)
   (xy 151.873161 70.717993) (xy 151.704112 70.677241) (xy 151.541996 70.63074) (xy 151.387039 70.578598) (xy 151.239467 70.520925)
   (xy 151.099507 70.457831) (xy 150.967385 70.389425) (xy 150.843329 70.315816) (xy 150.727564 70.237115) (xy 150.620318 70.153431)
   (xy 150.521817 70.064872) (xy 150.432287 69.97155) (xy 150.351955 69.873574) (xy 150.281047 69.771052) (xy 150.239903 69.703254)
   (xy 150.203083 69.636552) (xy 150.170436 69.569895) (xy 150.141808 69.502228) (xy 150.117043 69.432499) (xy 150.095989 69.359654)
   (xy 150.078492 69.282642) (xy 150.064398 69.200408) (xy 150.053553 69.111901) (xy 150.045804 69.016066) (xy 150.040997 68.911851)
   (xy 150.038978 68.798203) (xy 150.039593 68.674069) (xy 150.042688 68.538396) (xy 150.04811 68.39013) (xy 150.055705 68.22822)
   (xy 150.072415 67.962758) (xy 150.098332 67.715002) (xy 150.116664 67.59479) (xy 150.139604 67.475438) (xy 150.16792 67.355755)
   (xy 150.202381 67.234552) (xy 150.243756 67.110641) (xy 150.292814 66.982832) (xy 150.350322 66.849936) (xy 150.41705 66.710763)
   (xy 150.493766 66.564125) (xy 150.58124 66.408832) (xy 150.680239 66.243695) (xy 150.791532 66.067525) (xy 150.915888 65.879133)
   (xy 151.054076 65.677329) (xy 151.375022 65.228731) (xy 151.760519 64.712216) (xy 152.216716 64.11827) (xy 152.749763 63.437382)
   (xy 153.365808 62.660036) (xy 154.871494 60.777918) (xy 157.351611 57.70227) (xy 158.182147 56.694478) (xy 158.801918 55.969401)
   (xy 159.257611 55.474061) (xy 159.595914 55.15548) (xy 159.735634 55.045918) (xy 159.863513 54.960679) (xy 160.107097 54.83668)
   (xy 160.2199 54.793912) (xy 160.345893 54.756391) (xy 160.483077 54.724149) (xy 160.629452 54.697218) (xy 160.783018 54.67563)
   (xy 160.941774 54.659418) (xy 161.10372 54.648615) (xy 161.266857 54.643252))
  (stroke (width 0.1) (type solid)) (fill none) (layer "Edge.Cuts"))
 (segment (start 103.303266 85.851905) (end 103.319547 85.868186) (width 0.25) (layer "F.Cu") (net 3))
 (segment (start 102.746233 85.851905) (end 103.303266 85.851905) (width 0.25) (layer "F.Cu") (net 3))
 (segment (start 104.597733 84.59) (end 105.61 84.59) (width 0.25) (layer "F.Cu") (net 3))
 (segment (start 102.182894 89.488566) (end 102.182894 85.288566) (width 0.25) (layer "F.Cu") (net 3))
 (segment (start 103.319547 85.868186) (end 104.597733 84.59) (width 0.25) (layer "F.Cu") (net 3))
 (segment (start 102.182894 85.288566) (end 102.746233 85.851905) (width 0.25) (layer "F.Cu") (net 3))
 (segment (start 104.076952 82.05) (end 103.924584 82.202368) (width 0.25) (layer "F.Cu") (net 2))
 (segment (start 100.368882 81.636268) (end 102.411261 81.636268) (width 0.25) (layer "F.Cu") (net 2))
 (segment (start 105.61 82.05) (end 104.076952 82.05) (width 0.25) (layer "F.Cu") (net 2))
 (segment (start 103.358484 81.636268) (end 103.924584 82.202368) (width 0.25) (layer "F.Cu") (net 2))
 (segment (start 102.411261 81.636268) (end 103.358484 81.636268) (width 0.25) (layer "F.Cu") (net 2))
 (segment (start 103.319547 84.444554) (end 102.411261 83.536268) (width 0.25) (layer "F.Cu") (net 1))
 (segment (start 100.368882 83.536268) (end 102.411261 83.536268) (width 0.25) (layer "F.Cu") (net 1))
 (segment (start 104.082216 83.32) (end 103.924584 83.162368) (width 0.25) (layer "F.Cu") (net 1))
 (segment (start 102.785161 83.162368) (end 102.411261 83.536268) (width 0.25) (layer "F.Cu") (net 1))
 (segment (start 105.61 83.32) (end 104.082216 83.32) (width 0.25) (layer "F.Cu") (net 1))
 (segment (start 103.319547 84.848186) (end 103.319547 84.444554) (width 0.25) (layer "F.Cu") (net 1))
 (segment (start 103.924584 83.162368) (end 102.785161 83.162368) (width 0.25) (layer "F.Cu") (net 1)))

